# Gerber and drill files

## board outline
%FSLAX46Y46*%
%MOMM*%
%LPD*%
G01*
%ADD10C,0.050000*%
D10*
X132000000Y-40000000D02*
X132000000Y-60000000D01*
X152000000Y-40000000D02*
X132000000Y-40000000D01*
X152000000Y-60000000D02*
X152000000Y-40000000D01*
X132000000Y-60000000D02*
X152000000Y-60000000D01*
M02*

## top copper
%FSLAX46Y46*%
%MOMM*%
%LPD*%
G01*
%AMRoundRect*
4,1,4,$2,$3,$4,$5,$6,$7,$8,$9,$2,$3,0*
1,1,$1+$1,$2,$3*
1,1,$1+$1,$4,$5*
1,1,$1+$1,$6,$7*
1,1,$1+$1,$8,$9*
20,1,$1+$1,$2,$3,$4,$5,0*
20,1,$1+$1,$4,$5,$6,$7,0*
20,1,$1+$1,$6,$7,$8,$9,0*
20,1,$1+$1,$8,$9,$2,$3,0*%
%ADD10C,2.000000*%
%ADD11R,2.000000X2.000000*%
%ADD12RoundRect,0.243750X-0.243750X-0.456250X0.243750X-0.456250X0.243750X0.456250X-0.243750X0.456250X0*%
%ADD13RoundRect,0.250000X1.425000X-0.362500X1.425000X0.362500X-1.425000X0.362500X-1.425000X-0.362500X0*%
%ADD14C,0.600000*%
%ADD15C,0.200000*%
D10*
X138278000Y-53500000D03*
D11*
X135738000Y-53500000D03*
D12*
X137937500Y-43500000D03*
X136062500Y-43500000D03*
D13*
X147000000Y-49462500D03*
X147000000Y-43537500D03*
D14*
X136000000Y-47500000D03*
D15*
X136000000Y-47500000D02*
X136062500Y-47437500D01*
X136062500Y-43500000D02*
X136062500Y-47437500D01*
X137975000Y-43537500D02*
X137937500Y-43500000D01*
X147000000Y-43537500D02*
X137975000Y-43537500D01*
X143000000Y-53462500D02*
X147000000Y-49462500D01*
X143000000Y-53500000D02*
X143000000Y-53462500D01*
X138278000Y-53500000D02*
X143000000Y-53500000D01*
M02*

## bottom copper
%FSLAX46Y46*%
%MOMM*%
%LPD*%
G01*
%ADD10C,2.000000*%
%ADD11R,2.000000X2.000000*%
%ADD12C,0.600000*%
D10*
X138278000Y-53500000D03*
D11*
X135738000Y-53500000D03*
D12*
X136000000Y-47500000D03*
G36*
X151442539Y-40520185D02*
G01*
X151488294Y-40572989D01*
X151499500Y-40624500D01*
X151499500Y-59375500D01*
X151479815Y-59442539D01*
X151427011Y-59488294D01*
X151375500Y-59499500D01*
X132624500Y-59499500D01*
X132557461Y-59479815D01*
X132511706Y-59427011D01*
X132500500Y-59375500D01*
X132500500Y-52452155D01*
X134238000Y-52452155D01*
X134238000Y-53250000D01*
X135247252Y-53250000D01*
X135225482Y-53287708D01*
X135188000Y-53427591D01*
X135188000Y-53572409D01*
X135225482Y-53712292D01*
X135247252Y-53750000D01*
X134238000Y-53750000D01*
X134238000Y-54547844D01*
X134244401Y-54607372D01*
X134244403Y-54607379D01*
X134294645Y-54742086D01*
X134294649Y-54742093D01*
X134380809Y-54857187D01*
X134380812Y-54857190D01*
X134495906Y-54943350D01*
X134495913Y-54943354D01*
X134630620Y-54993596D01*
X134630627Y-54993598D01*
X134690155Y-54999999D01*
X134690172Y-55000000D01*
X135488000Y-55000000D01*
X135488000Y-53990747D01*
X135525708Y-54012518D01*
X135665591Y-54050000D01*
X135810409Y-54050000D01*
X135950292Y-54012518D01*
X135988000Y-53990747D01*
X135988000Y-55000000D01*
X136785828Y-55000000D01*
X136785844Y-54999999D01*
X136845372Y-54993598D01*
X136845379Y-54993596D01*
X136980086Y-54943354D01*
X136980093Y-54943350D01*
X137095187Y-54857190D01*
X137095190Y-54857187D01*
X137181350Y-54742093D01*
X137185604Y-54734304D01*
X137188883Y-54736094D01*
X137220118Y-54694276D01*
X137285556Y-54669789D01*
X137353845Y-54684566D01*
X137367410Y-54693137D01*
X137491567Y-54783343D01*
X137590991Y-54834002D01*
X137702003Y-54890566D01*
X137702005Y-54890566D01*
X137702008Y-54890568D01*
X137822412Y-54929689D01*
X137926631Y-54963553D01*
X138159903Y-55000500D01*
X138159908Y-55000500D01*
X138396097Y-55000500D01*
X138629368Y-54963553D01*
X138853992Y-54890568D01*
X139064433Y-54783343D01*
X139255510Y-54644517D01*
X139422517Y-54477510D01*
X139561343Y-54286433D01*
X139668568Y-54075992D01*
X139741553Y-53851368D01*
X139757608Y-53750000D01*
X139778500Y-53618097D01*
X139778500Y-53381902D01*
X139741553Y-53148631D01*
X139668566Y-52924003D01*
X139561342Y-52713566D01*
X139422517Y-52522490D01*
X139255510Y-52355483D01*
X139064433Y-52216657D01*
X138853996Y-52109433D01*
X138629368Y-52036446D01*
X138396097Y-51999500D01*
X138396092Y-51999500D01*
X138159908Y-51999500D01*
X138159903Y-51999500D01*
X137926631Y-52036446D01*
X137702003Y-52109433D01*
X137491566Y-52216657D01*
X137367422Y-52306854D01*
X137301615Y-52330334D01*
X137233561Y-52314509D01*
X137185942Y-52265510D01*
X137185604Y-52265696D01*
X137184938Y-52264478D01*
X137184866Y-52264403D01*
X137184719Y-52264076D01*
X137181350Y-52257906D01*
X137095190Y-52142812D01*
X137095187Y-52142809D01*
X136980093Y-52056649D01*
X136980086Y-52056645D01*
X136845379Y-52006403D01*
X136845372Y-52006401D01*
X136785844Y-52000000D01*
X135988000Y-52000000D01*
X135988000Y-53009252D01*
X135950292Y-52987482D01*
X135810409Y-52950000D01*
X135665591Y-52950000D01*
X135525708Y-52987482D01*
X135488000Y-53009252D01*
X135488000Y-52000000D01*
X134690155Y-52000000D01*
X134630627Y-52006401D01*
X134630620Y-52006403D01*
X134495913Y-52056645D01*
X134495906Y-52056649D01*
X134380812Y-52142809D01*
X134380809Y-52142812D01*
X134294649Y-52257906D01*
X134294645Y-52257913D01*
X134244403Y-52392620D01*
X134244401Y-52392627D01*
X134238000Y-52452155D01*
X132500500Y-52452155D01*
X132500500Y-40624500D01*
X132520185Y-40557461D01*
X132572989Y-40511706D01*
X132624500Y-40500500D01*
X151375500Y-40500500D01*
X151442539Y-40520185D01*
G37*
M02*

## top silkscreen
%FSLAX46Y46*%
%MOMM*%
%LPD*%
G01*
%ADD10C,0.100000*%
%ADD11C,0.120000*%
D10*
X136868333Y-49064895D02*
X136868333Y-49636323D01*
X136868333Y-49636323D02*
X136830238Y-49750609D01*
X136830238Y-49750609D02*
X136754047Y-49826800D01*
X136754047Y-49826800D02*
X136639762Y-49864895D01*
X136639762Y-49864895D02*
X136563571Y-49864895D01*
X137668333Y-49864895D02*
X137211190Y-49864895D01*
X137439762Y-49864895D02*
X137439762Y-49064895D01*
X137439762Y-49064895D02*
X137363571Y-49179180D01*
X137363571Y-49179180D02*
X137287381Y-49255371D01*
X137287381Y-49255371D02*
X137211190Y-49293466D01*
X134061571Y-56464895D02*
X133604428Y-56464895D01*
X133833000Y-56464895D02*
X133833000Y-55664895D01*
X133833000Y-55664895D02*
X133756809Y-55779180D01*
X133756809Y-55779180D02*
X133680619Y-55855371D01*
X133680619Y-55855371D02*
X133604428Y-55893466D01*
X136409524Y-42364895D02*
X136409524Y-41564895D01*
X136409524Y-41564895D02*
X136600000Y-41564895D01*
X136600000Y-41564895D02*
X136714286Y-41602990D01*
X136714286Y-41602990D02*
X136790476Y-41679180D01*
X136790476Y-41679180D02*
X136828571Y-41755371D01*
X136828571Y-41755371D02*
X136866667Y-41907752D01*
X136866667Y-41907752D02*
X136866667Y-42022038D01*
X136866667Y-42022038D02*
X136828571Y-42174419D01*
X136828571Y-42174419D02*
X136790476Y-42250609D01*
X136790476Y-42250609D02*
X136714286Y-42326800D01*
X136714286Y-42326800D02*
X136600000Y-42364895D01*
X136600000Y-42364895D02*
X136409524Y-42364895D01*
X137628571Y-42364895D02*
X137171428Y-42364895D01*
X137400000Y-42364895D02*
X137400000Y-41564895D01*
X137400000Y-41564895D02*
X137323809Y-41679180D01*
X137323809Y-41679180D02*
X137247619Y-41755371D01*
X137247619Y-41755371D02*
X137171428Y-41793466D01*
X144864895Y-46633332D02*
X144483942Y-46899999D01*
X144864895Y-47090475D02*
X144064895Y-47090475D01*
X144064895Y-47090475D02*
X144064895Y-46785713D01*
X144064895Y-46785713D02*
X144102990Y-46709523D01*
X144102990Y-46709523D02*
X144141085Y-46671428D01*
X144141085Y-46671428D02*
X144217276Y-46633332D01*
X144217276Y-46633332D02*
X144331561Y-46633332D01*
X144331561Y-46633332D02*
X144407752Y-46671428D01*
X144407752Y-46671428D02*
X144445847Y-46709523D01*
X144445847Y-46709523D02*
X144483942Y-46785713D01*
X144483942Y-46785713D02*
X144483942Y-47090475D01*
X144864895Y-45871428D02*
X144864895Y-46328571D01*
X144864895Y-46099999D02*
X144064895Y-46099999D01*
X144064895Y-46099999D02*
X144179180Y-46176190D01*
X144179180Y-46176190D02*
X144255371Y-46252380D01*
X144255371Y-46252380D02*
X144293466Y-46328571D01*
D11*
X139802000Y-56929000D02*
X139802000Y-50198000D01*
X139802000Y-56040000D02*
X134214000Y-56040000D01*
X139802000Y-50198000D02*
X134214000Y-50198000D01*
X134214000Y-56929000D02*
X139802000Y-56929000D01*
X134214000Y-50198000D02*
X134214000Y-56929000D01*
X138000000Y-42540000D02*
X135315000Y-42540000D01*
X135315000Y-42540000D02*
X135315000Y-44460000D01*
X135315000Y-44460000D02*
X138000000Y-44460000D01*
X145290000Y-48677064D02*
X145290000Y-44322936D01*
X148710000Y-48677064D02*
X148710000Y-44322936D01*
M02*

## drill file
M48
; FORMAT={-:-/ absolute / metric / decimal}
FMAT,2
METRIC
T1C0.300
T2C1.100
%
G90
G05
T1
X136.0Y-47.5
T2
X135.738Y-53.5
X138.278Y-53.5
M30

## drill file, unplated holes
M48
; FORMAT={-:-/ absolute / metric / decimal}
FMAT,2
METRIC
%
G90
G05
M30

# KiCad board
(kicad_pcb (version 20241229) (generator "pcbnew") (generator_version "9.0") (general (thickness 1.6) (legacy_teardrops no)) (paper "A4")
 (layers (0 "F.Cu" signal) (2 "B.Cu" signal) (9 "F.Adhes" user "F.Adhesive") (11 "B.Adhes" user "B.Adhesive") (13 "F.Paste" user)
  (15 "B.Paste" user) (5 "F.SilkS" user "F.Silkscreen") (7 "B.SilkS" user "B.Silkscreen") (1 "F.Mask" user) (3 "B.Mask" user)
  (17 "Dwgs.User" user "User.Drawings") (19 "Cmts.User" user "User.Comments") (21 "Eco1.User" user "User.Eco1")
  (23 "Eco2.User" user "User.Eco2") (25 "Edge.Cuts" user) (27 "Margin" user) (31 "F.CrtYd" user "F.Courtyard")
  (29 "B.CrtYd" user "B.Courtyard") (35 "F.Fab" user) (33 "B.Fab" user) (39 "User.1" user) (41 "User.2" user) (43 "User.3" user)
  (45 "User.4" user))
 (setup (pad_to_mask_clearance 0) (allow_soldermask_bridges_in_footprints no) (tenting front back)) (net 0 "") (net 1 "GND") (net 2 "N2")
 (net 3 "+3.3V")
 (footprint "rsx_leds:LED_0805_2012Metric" (layer "F.Cu") (at 137 43.5)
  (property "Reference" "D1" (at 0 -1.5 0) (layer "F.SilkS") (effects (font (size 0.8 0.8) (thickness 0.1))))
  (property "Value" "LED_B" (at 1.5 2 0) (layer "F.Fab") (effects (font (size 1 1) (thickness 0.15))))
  (fp_line (start -1.685 -0.96) (end -1.685 0.96) (stroke (width 0.12) (type solid)) (layer "F.SilkS"))
  (fp_line (start -1.685 0.96) (end 1 0.96) (stroke (width 0.12) (type solid)) (layer "F.SilkS"))
  (fp_line (start 1 -0.96) (end -1.685 -0.96) (stroke (width 0.12) (type solid)) (layer "F.SilkS"))
  (pad "1" smd roundrect (at -0.9375 0) (size 0.975 1.4) (layers "F.Cu" "F.Mask" "F.Paste") (roundrect_rratio 0.25) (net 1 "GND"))
  (pad "2" smd roundrect (at 0.9375 0) (size 0.975 1.4) (layers "F.Cu" "F.Mask" "F.Paste") (roundrect_rratio 0.25) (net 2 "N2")))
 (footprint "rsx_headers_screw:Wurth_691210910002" (layer "F.Cu") (at 136.5 53.5)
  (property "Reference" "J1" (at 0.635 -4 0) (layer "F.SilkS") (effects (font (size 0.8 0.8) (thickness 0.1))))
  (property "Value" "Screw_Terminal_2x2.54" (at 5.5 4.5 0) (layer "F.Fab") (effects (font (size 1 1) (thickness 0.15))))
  (fp_line (start -2.286 -3.302) (end -2.286 3.429) (stroke (width 0.12) (type solid)) (layer "F.SilkS"))
  (fp_line (start -2.286 3.429) (end 3.302 3.429) (stroke (width 0.12) (type solid)) (layer "F.SilkS"))
  (fp_line (start 3.302 -3.302) (end -2.286 -3.302) (stroke (width 0.12) (type solid)) (layer "F.SilkS"))
  (fp_line (start 3.302 2.54) (end -2.286 2.54) (stroke (width 0.12) (type solid)) (layer "F.SilkS"))
  (fp_line (start 3.302 3.429) (end 3.302 -3.302) (stroke (width 0.12) (type solid)) (layer "F.SilkS"))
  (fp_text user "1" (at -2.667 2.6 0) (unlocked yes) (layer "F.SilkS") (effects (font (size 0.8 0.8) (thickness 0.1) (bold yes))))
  (pad "1" thru_hole rect (at -0.762 0) (size 2 2) (drill 1.1) (layers "*.Cu" "*.Mask") (remove_unused_layers no) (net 1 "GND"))
  (pad "2" thru_hole circle (at 1.778 0) (size 2 2) (drill 1.1) (layers "*.Cu" "*.Mask") (remove_unused_layers no) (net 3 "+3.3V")))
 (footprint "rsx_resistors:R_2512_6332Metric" (layer "F.Cu") (at 147 46.5 90)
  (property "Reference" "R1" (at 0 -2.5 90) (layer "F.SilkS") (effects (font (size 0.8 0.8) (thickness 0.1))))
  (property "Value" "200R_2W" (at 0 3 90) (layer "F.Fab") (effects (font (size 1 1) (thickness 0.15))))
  (fp_line (start -2.177064 -1.71) (end 2.177064 -1.71) (stroke (width 0.12) (type solid)) (layer "F.SilkS"))
  (fp_line (start -2.177064 1.71) (end 2.177064 1.71) (stroke (width 0.12) (type solid)) (layer "F.SilkS"))
  (pad "1" smd roundrect (at -2.9625 0 90) (size 1.225 3.35) (layers "F.Cu" "F.Mask" "F.Paste") (roundrect_rratio 0.204082) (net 3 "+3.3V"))
  (pad "2" smd roundrect (at 2.9625 0 90) (size 1.225 3.35) (layers "F.Cu" "F.Mask" "F.Paste") (roundrect_rratio 0.204082) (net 2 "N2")))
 (gr_line (start 152 60) (end 152 40) (stroke (width 0.05) (type default)) (layer "Edge.Cuts"))
 (gr_line (start 132 60) (end 152 60) (stroke (width 0.05) (type default)) (layer "Edge.Cuts"))
 (gr_line (start 152 40) (end 132 40) (stroke (width 0.05) (type default)) (layer "Edge.Cuts"))
 (gr_line (start 132 40) (end 132 60) (stroke (width 0.05) (type default)) (layer "Edge.Cuts"))
 (segment (start 136 47.5) (end 136.0625 47.4375) (width 0.2) (layer "F.Cu") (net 1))
 (segment (start 136.0625 43.5) (end 136.0625 47.4375) (width 0.2) (layer "F.Cu") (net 1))
 (via (at 136 47.5) (size 0.6) (drill 0.3) (layers "F.Cu" "B.Cu") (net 1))
 (segment (start 147 43.5375) (end 137.975 43.5375) (width 0.2) (layer "F.Cu") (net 2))
 (segment (start 137.975 43.5375) (end 137.9375 43.5) (width 0.2) (layer "F.Cu") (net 2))
 (segment (start 143 53.5) (end 143 53.4625) (width 0.2) (layer "F.Cu") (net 3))
 (segment (start 143 53.4625) (end 147 49.4625) (width 0.2) (layer "F.Cu") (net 3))
 (segment (start 138.278 53.5) (end 143 53.5) (width 0.2) (layer "F.Cu") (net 3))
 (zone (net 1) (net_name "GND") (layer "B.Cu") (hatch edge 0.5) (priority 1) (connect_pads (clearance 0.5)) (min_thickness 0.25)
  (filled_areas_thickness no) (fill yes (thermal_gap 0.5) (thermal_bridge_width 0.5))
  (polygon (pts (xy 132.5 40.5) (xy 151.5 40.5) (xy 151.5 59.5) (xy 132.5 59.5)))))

